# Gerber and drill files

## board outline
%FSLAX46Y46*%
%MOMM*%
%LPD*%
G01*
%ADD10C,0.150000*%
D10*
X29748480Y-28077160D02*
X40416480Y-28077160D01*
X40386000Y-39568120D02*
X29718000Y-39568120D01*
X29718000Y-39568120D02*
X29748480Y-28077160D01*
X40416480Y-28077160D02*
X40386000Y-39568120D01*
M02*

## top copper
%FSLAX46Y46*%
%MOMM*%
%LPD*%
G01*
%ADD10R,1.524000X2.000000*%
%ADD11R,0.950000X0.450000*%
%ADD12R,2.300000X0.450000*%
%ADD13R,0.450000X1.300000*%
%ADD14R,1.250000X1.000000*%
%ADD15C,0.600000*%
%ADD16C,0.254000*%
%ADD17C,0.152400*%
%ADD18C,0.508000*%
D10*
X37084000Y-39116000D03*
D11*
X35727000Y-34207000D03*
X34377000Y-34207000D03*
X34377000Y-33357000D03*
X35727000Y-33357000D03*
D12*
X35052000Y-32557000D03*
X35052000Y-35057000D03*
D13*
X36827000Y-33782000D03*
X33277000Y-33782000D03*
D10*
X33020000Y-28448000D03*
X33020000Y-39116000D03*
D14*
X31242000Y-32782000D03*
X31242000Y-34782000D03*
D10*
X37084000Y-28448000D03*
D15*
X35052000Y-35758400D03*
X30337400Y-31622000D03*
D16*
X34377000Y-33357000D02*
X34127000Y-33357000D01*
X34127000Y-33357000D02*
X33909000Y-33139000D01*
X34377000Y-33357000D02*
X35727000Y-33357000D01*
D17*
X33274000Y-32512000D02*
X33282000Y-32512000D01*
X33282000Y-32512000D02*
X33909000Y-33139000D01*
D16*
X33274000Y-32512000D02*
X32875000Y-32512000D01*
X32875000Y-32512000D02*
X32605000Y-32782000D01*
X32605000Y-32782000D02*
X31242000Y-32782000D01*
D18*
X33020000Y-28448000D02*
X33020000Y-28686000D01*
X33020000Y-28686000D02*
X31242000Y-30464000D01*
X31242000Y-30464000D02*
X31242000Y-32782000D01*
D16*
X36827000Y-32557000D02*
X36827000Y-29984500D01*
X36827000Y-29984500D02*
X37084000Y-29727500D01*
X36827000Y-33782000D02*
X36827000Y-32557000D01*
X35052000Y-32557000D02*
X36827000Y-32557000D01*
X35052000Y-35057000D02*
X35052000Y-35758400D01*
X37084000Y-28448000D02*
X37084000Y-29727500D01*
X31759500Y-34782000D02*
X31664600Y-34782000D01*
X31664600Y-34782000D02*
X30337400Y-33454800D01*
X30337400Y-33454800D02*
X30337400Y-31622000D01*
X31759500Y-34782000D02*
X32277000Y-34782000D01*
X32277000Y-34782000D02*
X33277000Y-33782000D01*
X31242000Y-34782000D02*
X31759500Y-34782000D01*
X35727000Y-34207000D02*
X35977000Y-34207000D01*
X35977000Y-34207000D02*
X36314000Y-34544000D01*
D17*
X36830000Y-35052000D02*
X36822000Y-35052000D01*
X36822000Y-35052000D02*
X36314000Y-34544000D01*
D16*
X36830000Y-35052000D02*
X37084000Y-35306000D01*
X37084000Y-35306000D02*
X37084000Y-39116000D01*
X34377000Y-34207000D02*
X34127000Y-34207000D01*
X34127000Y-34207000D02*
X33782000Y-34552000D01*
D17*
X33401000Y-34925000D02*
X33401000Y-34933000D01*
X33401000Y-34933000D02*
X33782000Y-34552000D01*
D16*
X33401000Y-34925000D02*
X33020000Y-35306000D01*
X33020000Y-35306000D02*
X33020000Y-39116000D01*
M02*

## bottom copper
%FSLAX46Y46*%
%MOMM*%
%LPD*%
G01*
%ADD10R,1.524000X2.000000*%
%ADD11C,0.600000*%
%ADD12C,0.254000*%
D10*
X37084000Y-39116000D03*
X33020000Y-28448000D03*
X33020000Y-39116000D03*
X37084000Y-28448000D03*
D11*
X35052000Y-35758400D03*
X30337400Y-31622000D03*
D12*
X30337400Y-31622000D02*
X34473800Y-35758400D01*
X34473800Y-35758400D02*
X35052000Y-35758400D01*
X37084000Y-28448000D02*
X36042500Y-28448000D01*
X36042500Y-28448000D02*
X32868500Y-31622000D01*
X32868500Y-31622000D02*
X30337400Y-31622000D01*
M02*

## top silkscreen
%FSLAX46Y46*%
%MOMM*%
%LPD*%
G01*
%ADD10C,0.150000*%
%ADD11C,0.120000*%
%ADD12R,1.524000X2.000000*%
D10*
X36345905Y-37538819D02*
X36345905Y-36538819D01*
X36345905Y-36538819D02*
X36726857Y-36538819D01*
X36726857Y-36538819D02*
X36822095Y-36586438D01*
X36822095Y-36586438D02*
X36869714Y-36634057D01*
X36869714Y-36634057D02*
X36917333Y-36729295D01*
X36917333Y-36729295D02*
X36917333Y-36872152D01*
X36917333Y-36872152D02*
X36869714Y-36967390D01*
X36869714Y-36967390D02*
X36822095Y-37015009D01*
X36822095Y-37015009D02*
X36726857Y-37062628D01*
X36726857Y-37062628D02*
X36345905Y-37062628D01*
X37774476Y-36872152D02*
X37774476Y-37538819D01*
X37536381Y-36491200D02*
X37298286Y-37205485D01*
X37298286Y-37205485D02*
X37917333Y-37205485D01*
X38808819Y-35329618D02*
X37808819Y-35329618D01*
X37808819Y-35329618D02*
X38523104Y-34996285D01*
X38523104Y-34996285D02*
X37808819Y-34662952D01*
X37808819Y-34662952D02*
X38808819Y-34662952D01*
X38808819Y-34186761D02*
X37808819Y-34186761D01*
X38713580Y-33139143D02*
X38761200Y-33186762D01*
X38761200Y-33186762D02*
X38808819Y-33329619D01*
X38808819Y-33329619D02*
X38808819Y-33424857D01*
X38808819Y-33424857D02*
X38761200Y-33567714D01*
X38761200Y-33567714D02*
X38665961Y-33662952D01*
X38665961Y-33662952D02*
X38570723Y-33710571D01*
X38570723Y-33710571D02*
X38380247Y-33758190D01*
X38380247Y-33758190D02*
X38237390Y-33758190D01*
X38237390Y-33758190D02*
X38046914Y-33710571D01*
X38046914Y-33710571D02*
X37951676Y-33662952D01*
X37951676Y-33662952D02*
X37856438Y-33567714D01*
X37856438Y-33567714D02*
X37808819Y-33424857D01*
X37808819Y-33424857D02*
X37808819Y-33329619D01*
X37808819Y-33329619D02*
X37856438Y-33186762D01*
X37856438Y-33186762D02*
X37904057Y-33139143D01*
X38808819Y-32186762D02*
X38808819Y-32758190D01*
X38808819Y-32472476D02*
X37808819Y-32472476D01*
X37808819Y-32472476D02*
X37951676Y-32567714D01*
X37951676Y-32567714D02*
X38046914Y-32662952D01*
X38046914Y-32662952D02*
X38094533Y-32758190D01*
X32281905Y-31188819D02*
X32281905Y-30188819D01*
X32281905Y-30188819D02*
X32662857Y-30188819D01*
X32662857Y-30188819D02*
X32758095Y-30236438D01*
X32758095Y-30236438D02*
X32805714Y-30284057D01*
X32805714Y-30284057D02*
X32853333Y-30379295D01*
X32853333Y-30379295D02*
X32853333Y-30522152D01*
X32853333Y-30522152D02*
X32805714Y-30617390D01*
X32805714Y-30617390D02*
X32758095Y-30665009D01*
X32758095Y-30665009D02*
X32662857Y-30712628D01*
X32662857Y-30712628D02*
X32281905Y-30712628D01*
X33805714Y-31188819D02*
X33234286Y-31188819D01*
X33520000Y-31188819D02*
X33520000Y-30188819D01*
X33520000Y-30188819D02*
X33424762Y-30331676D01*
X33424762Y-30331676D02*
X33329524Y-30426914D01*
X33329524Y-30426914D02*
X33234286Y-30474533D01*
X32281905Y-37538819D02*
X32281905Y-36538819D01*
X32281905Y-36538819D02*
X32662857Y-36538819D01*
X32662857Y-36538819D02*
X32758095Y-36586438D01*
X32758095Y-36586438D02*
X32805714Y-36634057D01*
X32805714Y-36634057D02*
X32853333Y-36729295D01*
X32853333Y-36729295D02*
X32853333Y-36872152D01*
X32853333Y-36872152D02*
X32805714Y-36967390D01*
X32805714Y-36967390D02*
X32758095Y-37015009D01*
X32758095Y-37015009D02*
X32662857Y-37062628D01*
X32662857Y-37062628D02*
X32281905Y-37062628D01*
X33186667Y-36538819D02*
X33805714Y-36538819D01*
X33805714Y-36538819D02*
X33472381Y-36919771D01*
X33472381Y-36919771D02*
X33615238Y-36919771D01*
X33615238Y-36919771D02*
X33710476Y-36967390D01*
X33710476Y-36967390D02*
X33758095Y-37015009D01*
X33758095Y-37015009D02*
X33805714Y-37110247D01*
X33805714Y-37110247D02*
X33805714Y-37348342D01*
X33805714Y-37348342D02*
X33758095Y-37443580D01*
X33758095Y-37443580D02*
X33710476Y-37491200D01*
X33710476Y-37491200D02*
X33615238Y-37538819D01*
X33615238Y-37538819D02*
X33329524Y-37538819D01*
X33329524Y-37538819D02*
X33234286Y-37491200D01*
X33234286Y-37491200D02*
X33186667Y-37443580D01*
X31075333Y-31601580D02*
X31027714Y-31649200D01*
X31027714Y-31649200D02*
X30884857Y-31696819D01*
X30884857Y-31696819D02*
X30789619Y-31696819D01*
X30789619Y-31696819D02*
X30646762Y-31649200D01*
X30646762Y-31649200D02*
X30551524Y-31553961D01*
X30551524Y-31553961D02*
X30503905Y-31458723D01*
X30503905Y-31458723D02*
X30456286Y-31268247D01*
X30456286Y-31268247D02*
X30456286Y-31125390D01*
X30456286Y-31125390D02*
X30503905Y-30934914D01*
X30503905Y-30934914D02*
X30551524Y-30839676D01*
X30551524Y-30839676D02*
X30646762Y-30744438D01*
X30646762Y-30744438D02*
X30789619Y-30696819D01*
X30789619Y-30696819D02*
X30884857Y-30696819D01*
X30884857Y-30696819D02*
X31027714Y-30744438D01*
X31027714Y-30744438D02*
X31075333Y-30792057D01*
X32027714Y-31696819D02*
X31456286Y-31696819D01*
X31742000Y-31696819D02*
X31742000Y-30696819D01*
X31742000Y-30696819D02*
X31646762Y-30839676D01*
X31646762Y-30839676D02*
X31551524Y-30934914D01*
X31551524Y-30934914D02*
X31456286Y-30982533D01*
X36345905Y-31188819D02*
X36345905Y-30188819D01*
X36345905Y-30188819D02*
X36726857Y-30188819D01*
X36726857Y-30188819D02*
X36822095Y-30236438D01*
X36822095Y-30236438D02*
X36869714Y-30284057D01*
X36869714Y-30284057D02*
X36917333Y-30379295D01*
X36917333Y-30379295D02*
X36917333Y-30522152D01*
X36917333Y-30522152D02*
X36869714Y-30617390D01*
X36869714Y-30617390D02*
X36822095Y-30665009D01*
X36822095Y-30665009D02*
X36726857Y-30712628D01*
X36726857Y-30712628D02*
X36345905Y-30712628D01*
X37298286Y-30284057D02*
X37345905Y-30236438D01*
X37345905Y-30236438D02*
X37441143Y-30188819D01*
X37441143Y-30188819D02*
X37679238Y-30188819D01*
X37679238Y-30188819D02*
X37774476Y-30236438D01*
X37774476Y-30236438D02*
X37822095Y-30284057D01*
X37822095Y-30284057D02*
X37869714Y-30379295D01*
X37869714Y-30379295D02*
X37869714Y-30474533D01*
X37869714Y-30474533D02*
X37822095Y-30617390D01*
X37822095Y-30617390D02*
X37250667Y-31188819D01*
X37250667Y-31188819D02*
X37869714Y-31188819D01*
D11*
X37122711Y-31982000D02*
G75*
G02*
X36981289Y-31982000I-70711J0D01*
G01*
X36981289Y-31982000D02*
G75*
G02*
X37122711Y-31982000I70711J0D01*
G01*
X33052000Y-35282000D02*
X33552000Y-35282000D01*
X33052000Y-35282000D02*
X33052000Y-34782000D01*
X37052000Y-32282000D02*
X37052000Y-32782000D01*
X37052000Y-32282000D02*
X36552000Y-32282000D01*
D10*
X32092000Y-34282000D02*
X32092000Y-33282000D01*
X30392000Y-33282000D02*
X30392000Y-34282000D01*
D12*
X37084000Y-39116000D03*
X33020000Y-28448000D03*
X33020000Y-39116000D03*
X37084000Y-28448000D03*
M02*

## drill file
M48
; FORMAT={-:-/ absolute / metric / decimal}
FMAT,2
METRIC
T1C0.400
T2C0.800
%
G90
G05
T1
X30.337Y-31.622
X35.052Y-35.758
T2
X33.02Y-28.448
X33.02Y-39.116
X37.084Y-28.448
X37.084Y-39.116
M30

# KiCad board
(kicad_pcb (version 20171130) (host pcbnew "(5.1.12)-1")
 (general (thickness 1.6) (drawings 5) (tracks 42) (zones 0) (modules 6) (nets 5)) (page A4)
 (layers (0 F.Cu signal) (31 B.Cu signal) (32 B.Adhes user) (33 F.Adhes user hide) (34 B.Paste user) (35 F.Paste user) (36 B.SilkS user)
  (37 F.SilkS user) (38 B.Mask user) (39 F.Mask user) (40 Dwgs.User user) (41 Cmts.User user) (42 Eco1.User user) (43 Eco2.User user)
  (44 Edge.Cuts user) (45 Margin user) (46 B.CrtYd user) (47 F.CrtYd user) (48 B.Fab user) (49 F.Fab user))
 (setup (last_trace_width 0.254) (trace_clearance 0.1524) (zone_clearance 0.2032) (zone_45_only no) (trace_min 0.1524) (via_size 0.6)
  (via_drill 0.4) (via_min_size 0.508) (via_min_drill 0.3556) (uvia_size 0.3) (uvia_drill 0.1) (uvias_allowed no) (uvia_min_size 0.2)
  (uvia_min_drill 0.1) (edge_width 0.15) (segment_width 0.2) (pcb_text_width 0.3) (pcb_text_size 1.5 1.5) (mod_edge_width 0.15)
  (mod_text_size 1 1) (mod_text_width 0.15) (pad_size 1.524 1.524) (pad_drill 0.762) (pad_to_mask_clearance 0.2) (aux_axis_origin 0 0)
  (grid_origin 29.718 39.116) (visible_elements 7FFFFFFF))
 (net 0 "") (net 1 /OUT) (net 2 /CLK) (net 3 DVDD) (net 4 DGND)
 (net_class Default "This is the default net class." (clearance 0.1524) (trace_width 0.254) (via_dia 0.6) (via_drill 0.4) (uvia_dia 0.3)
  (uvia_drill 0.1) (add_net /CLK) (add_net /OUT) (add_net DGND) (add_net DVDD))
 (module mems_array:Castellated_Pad (layer F.Cu) (at 37.084 39.116)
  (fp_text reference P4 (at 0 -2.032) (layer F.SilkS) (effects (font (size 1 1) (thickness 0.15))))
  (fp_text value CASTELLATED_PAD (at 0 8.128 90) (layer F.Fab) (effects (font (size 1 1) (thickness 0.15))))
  (pad 1 thru_hole rect (at 0 0) (size 1.524 2) (drill 0.8) (layers *.Cu *.Mask F.SilkS) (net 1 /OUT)))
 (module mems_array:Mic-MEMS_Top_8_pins (layer F.Cu) (at 35.052 33.782 90)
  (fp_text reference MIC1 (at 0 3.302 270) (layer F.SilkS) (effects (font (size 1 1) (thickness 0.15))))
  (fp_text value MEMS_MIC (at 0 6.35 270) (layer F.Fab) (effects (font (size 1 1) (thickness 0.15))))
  (fp_circle (center 1.8 2) (end 1.85 2.05) (layer F.SilkS) (width 0.12))
  (fp_line (start -1.5 -2) (end -1.5 -1.5) (layer F.SilkS) (width 0.12))
  (fp_line (start -1.5 -2) (end -1 -2) (layer F.SilkS) (width 0.12))
  (fp_line (start 1.5 2) (end 1 2) (layer F.SilkS) (width 0.12))
  (fp_line (start 1.5 2) (end 1.5 1.5) (layer F.SilkS) (width 0.12))
  (pad 4 smd rect (at -0.425 0.675 90) (size 0.45 0.95) (layers F.Cu F.Paste F.Mask) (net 1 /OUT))
  (pad 3 smd rect (at -0.425 -0.675 90) (size 0.45 0.95) (layers F.Cu F.Paste F.Mask) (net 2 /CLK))
  (pad 2 smd rect (at 0.425 -0.675 90) (size 0.45 0.95) (layers F.Cu F.Paste F.Mask) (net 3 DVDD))
  (pad 1 smd rect (at 0.425 0.675 90) (size 0.45 0.95) (layers F.Cu F.Paste F.Mask) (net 3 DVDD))
  (pad 5 smd rect (at 1.225 0 90) (size 0.45 2.3) (layers F.Cu F.Paste F.Mask) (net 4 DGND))
  (pad 5 smd rect (at -1.275 0 90) (size 0.45 2.3) (layers F.Cu F.Paste F.Mask) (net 4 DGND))
  (pad 5 smd rect (at 0 1.775 90) (size 1.3 0.45) (layers F.Cu F.Paste F.Mask) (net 4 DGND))
  (pad 5 smd rect (at 0 -1.775 90) (size 1.3 0.45) (layers F.Cu F.Paste F.Mask) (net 4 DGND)))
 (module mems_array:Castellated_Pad (layer F.Cu) (at 33.02 28.448)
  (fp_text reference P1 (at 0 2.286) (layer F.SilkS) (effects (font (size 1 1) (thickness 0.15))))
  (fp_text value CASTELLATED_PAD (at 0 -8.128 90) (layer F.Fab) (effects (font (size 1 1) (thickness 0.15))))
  (pad 1 thru_hole rect (at 0 0) (size 1.524 2) (drill 0.8) (layers *.Cu *.Mask F.SilkS) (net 3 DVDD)))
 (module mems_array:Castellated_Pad (layer F.Cu) (at 33.02 39.116)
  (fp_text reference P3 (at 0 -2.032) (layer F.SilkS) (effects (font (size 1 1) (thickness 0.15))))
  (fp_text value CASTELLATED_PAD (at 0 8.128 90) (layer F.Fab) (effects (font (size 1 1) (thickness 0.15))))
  (pad 1 thru_hole rect (at 0 0) (size 1.524 2) (drill 0.8) (layers *.Cu *.Mask F.SilkS) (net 2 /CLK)))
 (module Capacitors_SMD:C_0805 (layer F.Cu) (at 31.242 33.782 270)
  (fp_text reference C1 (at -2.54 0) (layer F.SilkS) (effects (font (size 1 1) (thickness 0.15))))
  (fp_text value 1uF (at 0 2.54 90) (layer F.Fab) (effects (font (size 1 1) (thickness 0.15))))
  (fp_line (start 0.5 -0.85) (end -0.5 -0.85) (layer F.SilkS) (width 0.15))
  (fp_line (start -0.5 0.85) (end 0.5 0.85) (layer F.SilkS) (width 0.15))
  (pad 1 smd rect (at -1 0 270) (size 1 1.25) (layers F.Cu F.Paste F.Mask) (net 3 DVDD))
  (pad 2 smd rect (at 1 0 270) (size 1 1.25) (layers F.Cu F.Paste F.Mask) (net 4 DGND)))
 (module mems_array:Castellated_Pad (layer F.Cu) (at 37.084 28.448)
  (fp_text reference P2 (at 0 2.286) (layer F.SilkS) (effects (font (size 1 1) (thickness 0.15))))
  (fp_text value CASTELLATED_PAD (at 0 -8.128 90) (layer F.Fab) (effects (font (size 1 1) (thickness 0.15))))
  (pad 1 thru_hole rect (at 0 0) (size 1.524 2) (drill 0.8) (layers *.Cu *.Mask F.SilkS) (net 4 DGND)))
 (gr_line (start 29.74848 28.07716) (end 40.41648 28.07716) (layer Edge.Cuts) (width 0.15))
 (gr_line (start 40.386 39.56812) (end 29.718 39.56812) (layer Edge.Cuts) (width 0.15))
 (gr_line (start 29.718 39.56812) (end 29.74848 28.07716) (layer Edge.Cuts) (width 0.15))
 (gr_line (start 40.41648 28.07716) (end 40.386 39.56812) (layer Edge.Cuts) (width 0.15))
 (segment (start 34.377 33.357) (end 34.127 33.357) (width 0.254) (layer F.Cu) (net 3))
 (segment (start 34.127 33.357) (end 33.909 33.139) (width 0.254) (layer F.Cu) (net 3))
 (segment (start 34.377 33.357) (end 35.727 33.357) (width 0.254) (layer F.Cu) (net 3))
 (segment (start 33.274 32.512) (end 33.282 32.512) (width 0.1524) (layer F.Cu) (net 3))
 (segment (start 33.282 32.512) (end 33.909 33.139) (width 0.1524) (layer F.Cu) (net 3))
 (segment (start 33.274 32.512) (end 32.875 32.512) (width 0.254) (layer F.Cu) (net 3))
 (segment (start 32.875 32.512) (end 32.605 32.782) (width 0.254) (layer F.Cu) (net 3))
 (segment (start 32.605 32.782) (end 31.242 32.782) (width 0.254) (layer F.Cu) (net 3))
 (segment (start 33.02 28.448) (end 33.02 28.686) (width 0.508) (layer F.Cu) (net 3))
 (segment (start 33.02 28.686) (end 31.242 30.464) (width 0.508) (layer F.Cu) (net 3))
 (segment (start 31.242 30.464) (end 31.242 32.782) (width 0.508) (layer F.Cu) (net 3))
 (segment (start 36.827 32.557) (end 36.827 29.9845) (width 0.254) (layer F.Cu) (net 4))
 (segment (start 36.827 29.9845) (end 37.084 29.7275) (width 0.254) (layer F.Cu) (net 4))
 (segment (start 36.827 33.782) (end 36.827 32.557) (width 0.254) (layer F.Cu) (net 4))
 (segment (start 35.052 32.557) (end 36.827 32.557) (width 0.254) (layer F.Cu) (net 4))
 (segment (start 35.052 35.057) (end 35.052 35.7584) (width 0.254) (layer F.Cu) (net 4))
 (segment (start 30.3374 31.622) (end 34.4738 35.7584) (width 0.254) (layer B.Cu) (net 4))
 (segment (start 34.4738 35.7584) (end 35.052 35.7584) (width 0.254) (layer B.Cu) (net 4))
 (segment (start 37.084 28.448) (end 37.084 29.7275) (width 0.254) (layer F.Cu) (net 4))
 (segment (start 37.084 28.448) (end 36.0425 28.448) (width 0.254) (layer B.Cu) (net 4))
 (segment (start 31.7595 34.782) (end 31.6646 34.782) (width 0.254) (layer F.Cu) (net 4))
 (segment (start 31.6646 34.782) (end 30.3374 33.4548) (width 0.254) (layer F.Cu) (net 4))
 (segment (start 30.3374 33.4548) (end 30.3374 31.622) (width 0.254) (layer F.Cu) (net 4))
 (segment (start 36.0425 28.448) (end 32.8685 31.622) (width 0.254) (layer B.Cu) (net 4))
 (segment (start 32.8685 31.622) (end 30.3374 31.622) (width 0.254) (layer B.Cu) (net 4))
 (segment (start 31.7595 34.782) (end 32.277 34.782) (width 0.254) (layer F.Cu) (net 4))
 (segment (start 32.277 34.782) (end 33.277 33.782) (width 0.254) (layer F.Cu) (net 4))
 (segment (start 31.242 34.782) (end 31.7595 34.782) (width 0.254) (layer F.Cu) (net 4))
 (via (at 35.052 35.7584) (size 0.6) (layers F.Cu B.Cu) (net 4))
 (via (at 30.3374 31.622) (size 0.6) (layers F.Cu B.Cu) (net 4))
 (segment (start 35.727 34.207) (end 35.977 34.207) (width 0.254) (layer F.Cu) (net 1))
 (segment (start 35.977 34.207) (end 36.314 34.544) (width 0.254) (layer F.Cu) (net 1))
 (segment (start 36.83 35.052) (end 36.822 35.052) (width 0.1524) (layer F.Cu) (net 1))
 (segment (start 36.822 35.052) (end 36.314 34.544) (width 0.1524) (layer F.Cu) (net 1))
 (segment (start 36.83 35.052) (end 37.084 35.306) (width 0.254) (layer F.Cu) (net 1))
 (segment (start 37.084 35.306) (end 37.084 39.116) (width 0.254) (layer F.Cu) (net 1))
 (segment (start 34.377 34.207) (end 34.127 34.207) (width 0.254) (layer F.Cu) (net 2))
 (segment (start 34.127 34.207) (end 33.782 34.552) (width 0.254) (layer F.Cu) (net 2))
 (segment (start 33.401 34.925) (end 33.401 34.933) (width 0.1524) (layer F.Cu) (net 2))
 (segment (start 33.401 34.933) (end 33.782 34.552) (width 0.1524) (layer F.Cu) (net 2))
 (segment (start 33.401 34.925) (end 33.02 35.306) (width 0.254) (layer F.Cu) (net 2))
 (segment (start 33.02 35.306) (end 33.02 39.116) (width 0.254) (layer F.Cu) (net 2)))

